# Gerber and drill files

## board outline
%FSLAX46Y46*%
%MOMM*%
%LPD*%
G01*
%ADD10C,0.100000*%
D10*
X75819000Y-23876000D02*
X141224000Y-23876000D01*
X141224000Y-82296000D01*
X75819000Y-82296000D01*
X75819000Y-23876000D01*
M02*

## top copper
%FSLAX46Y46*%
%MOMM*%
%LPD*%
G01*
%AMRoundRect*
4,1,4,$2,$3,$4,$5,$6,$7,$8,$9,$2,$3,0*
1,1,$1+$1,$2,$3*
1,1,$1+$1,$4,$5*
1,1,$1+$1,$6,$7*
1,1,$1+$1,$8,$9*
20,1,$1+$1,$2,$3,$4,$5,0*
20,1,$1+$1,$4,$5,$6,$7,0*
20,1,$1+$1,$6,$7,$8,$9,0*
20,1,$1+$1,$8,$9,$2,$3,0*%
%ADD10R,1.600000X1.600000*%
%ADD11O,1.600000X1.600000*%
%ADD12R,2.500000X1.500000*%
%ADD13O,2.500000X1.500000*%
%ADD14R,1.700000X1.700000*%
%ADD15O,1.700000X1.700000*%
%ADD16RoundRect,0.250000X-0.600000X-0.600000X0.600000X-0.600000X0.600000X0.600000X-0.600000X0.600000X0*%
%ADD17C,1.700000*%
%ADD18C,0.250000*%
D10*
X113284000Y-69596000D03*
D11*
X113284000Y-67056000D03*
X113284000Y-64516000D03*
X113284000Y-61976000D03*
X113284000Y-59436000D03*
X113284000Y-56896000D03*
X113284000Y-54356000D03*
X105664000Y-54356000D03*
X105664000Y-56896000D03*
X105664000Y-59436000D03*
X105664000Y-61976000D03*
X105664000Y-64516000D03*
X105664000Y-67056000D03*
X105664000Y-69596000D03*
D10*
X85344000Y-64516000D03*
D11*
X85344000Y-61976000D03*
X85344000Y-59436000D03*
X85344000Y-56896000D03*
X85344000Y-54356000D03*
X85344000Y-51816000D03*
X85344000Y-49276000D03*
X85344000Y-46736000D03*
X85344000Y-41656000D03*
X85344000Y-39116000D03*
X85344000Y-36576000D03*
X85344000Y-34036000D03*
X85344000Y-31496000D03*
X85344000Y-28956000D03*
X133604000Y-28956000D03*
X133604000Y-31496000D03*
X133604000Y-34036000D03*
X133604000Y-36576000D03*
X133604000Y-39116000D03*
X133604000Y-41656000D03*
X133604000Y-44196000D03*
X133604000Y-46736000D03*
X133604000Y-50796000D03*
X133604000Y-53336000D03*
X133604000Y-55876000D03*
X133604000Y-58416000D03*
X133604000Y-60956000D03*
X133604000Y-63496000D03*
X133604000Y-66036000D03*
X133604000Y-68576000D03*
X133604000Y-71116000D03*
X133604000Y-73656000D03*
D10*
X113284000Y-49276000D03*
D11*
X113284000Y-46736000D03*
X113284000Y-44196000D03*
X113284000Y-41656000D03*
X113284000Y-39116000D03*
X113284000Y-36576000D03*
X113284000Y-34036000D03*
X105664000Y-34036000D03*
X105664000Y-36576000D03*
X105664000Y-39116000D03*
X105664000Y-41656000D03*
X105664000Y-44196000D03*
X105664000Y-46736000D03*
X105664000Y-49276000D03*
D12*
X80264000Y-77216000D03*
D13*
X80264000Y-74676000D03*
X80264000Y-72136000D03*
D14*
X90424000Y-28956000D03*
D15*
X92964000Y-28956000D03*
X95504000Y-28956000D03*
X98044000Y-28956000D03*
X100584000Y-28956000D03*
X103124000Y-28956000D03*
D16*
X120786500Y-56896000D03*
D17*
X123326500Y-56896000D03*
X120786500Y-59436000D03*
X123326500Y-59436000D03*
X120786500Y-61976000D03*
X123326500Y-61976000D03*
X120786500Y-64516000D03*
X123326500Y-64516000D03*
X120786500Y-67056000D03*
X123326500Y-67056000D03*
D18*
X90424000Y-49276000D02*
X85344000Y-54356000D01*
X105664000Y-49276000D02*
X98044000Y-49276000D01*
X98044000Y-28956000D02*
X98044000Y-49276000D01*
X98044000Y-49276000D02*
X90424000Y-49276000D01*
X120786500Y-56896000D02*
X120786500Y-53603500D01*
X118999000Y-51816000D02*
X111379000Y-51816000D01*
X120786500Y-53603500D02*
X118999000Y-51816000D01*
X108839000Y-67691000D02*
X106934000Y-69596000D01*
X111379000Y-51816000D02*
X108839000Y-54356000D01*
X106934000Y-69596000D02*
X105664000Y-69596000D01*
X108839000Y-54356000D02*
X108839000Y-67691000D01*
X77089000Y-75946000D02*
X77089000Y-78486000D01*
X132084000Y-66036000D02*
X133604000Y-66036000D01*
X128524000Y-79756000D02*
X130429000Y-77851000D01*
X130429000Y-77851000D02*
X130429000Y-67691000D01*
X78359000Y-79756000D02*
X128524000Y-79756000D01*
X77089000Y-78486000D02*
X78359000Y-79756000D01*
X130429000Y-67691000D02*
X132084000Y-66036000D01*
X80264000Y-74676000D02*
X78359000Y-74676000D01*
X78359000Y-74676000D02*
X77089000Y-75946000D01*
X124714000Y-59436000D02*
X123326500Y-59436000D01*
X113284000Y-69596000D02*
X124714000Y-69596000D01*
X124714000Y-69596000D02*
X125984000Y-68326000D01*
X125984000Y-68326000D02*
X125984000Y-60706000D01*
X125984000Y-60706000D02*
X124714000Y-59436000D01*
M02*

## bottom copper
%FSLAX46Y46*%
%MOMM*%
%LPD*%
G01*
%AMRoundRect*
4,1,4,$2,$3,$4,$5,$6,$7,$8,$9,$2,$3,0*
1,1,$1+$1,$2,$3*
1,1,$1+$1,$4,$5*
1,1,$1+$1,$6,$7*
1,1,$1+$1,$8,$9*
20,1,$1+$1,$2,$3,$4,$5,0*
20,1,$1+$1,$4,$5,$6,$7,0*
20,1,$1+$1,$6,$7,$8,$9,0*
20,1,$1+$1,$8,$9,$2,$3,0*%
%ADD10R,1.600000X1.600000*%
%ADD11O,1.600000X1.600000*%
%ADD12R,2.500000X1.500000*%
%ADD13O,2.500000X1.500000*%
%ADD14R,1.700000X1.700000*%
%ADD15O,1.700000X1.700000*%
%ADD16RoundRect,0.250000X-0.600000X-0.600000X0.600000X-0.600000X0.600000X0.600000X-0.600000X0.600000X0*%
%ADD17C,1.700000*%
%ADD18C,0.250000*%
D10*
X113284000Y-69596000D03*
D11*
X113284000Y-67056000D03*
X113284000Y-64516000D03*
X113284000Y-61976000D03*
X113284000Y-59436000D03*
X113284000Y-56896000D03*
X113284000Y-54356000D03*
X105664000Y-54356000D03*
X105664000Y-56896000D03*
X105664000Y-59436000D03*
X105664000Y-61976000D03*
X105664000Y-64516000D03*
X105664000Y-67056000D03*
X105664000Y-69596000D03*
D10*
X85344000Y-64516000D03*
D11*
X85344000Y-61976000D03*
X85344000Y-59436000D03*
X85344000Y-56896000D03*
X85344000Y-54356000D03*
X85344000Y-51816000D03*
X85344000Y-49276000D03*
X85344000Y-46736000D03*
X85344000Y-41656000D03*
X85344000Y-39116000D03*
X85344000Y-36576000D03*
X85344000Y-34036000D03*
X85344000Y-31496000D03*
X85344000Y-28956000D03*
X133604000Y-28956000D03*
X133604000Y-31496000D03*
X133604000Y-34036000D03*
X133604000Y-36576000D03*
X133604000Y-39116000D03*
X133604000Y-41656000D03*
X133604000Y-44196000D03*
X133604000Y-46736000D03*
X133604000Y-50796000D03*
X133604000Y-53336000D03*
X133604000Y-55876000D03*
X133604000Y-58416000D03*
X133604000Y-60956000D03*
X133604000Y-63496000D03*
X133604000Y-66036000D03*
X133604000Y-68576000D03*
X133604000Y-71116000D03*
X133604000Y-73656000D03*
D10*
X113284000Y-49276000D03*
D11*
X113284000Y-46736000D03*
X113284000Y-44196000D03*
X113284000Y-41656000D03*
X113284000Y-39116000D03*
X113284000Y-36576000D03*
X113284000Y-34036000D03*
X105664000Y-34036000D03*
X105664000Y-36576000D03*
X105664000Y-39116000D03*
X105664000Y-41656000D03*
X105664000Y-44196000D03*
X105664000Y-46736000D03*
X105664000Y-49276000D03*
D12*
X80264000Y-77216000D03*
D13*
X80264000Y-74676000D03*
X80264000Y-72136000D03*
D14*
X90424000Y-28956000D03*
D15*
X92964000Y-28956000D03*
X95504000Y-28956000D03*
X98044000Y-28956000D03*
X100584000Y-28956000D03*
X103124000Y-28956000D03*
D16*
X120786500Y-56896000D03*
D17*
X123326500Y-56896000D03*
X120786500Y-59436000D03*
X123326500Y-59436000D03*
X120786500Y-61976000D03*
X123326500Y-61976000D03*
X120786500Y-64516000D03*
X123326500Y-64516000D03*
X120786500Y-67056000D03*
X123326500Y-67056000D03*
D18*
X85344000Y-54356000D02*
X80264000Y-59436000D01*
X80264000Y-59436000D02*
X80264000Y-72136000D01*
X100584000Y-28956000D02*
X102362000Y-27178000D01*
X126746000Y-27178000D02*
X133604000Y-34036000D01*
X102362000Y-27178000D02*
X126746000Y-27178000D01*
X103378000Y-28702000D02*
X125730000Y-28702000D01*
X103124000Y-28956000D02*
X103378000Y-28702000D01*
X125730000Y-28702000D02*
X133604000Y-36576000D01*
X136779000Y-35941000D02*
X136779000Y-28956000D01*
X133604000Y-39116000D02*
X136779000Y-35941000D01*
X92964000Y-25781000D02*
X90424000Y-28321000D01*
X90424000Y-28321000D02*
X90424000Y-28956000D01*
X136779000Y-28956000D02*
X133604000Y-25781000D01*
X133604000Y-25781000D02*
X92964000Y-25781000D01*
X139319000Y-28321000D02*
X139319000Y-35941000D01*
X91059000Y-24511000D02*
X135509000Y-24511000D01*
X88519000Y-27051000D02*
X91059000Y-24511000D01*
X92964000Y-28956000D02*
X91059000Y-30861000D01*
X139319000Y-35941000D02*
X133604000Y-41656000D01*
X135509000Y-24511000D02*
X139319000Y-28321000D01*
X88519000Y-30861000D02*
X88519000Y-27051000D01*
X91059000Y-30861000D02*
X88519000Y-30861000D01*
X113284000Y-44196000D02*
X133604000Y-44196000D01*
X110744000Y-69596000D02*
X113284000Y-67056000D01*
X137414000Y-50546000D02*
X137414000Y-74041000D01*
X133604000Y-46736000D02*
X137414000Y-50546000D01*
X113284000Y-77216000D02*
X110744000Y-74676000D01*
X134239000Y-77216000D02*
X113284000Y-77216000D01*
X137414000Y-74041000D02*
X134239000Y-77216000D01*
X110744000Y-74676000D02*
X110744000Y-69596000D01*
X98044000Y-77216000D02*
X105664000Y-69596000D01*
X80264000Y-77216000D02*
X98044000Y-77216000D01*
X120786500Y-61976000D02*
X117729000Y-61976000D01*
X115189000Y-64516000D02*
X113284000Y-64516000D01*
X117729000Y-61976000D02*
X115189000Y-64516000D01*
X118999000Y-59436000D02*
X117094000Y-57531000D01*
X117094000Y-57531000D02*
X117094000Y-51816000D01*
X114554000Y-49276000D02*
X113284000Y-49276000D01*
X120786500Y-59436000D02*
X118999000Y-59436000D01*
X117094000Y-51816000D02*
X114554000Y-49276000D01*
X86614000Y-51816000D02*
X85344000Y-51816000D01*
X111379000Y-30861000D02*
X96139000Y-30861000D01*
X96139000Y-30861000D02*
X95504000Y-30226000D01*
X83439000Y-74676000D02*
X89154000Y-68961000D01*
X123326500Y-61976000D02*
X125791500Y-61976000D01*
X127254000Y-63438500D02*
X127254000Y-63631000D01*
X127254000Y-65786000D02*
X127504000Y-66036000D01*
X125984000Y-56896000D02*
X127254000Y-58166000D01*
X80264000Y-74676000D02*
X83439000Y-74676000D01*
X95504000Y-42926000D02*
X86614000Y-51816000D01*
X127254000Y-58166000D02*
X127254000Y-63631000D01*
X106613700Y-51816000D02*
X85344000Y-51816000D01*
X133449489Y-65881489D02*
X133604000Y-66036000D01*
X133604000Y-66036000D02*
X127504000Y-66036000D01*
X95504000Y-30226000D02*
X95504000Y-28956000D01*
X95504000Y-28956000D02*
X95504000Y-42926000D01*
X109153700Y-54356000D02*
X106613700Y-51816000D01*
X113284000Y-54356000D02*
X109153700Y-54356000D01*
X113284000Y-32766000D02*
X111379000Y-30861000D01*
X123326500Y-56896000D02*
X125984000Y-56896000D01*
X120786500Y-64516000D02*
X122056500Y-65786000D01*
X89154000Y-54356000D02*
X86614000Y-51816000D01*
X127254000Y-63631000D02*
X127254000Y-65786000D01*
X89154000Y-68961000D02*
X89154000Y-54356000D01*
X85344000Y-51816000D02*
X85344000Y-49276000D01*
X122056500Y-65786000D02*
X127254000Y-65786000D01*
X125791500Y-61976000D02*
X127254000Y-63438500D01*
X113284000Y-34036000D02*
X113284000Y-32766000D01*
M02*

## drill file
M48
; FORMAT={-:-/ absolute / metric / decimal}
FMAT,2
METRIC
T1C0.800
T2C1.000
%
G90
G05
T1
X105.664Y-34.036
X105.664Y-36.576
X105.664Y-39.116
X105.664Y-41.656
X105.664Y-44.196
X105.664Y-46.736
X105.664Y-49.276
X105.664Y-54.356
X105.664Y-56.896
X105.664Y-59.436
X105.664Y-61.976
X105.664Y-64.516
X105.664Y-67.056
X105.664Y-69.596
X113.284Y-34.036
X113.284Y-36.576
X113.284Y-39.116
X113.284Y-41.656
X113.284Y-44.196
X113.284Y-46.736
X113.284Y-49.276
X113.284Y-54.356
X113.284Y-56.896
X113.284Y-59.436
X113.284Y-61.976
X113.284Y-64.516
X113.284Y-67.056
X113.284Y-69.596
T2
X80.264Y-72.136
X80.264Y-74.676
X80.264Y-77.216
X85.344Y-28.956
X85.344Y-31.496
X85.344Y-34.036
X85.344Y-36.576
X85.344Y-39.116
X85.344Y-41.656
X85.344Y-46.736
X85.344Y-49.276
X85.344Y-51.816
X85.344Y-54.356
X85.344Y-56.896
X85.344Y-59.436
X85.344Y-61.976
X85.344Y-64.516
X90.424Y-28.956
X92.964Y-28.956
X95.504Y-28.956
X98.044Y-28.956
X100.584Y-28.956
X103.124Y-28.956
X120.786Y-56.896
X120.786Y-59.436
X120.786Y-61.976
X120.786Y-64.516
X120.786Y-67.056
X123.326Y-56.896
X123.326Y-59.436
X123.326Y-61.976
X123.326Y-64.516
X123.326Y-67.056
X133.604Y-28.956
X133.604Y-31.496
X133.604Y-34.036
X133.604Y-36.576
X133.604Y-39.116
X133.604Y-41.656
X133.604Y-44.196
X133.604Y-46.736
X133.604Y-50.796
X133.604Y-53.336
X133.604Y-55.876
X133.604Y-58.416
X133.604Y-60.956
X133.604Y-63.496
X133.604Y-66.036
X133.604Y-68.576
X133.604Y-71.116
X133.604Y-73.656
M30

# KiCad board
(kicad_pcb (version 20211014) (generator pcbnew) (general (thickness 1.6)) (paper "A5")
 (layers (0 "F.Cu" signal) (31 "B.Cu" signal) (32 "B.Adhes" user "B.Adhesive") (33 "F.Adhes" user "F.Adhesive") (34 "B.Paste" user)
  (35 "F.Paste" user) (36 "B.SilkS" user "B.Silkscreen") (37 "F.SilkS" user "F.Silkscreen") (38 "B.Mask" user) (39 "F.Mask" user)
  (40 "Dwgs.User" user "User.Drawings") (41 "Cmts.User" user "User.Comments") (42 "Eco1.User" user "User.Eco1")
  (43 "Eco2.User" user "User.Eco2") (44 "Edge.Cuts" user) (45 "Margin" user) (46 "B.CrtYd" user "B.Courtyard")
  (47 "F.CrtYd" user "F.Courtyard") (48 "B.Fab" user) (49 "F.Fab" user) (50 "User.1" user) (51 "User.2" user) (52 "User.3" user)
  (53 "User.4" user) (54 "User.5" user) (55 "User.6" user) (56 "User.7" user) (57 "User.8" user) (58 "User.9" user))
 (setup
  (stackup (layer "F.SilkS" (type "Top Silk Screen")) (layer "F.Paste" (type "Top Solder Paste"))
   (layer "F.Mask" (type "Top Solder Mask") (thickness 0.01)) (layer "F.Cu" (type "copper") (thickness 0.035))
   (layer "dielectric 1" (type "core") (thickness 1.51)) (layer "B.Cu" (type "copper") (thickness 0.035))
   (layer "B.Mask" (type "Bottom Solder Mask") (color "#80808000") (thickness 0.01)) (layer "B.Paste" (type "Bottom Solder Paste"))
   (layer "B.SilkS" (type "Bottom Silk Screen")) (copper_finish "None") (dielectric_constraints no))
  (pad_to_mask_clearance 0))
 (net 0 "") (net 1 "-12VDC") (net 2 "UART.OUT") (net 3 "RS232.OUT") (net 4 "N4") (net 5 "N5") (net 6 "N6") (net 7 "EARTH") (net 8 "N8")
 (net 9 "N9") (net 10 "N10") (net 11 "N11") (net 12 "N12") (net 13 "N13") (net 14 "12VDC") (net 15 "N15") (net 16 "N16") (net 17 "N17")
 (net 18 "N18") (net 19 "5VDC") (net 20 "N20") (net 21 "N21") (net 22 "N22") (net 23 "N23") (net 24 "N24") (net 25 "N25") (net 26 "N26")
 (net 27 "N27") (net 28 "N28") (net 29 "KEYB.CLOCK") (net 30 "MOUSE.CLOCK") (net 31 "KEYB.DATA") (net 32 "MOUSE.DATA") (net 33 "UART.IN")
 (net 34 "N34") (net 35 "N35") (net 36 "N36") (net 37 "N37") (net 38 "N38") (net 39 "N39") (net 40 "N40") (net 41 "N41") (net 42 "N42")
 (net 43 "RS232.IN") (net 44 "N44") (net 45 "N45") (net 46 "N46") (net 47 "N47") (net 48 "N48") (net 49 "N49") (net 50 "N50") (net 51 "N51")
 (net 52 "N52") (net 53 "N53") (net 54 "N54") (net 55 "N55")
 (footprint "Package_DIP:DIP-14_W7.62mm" (layer "F.Cu") (at 113.284 69.596 180)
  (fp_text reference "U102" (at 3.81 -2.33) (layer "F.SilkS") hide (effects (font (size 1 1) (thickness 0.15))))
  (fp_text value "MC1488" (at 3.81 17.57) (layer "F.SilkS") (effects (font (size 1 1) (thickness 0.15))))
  (pad "1" thru_hole rect (at 0 0 180) (size 1.6 1.6) (drill 0.8) (layers *.Cu *.Mask) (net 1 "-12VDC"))
  (pad "2" thru_hole oval (at 0 2.54 180) (size 1.6 1.6) (drill 0.8) (layers *.Cu *.Mask) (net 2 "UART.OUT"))
  (pad "3" thru_hole oval (at 0 5.08 180) (size 1.6 1.6) (drill 0.8) (layers *.Cu *.Mask) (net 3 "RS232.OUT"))
  (pad "4" thru_hole oval (at 0 7.62 180) (size 1.6 1.6) (drill 0.8) (layers *.Cu *.Mask) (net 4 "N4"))
  (pad "5" thru_hole oval (at 0 10.16 180) (size 1.6 1.6) (drill 0.8) (layers *.Cu *.Mask) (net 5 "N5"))
  (pad "6" thru_hole oval (at 0 12.7 180) (size 1.6 1.6) (drill 0.8) (layers *.Cu *.Mask) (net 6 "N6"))
  (pad "7" thru_hole oval (at 0 15.24 180) (size 1.6 1.6) (drill 0.8) (layers *.Cu *.Mask) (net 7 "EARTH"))
  (pad "8" thru_hole oval (at 7.62 15.24 180) (size 1.6 1.6) (drill 0.8) (layers *.Cu *.Mask) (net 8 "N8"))
  (pad "9" thru_hole oval (at 7.62 12.7 180) (size 1.6 1.6) (drill 0.8) (layers *.Cu *.Mask) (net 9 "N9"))
  (pad "10" thru_hole oval (at 7.62 10.16 180) (size 1.6 1.6) (drill 0.8) (layers *.Cu *.Mask) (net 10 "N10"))
  (pad "11" thru_hole oval (at 7.62 7.62 180) (size 1.6 1.6) (drill 0.8) (layers *.Cu *.Mask) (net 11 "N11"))
  (pad "12" thru_hole oval (at 7.62 5.08 180) (size 1.6 1.6) (drill 0.8) (layers *.Cu *.Mask) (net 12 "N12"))
  (pad "13" thru_hole oval (at 7.62 2.54 180) (size 1.6 1.6) (drill 0.8) (layers *.Cu *.Mask) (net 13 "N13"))
  (pad "14" thru_hole oval (at 7.62 0 180) (size 1.6 1.6) (drill 0.8) (layers *.Cu *.Mask) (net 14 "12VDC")))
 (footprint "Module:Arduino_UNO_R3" (layer "F.Cu") (at 85.344 64.516 90)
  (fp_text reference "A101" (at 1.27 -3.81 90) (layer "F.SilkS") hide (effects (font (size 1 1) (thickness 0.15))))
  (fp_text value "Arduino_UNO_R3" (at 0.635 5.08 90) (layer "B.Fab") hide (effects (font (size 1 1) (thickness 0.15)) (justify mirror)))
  (pad "1" thru_hole rect (at 0 0 180) (size 1.6 1.6) (drill 1) (layers *.Cu *.Mask) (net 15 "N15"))
  (pad "2" thru_hole oval (at 2.54 0 180) (size 1.6 1.6) (drill 1) (layers *.Cu *.Mask) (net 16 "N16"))
  (pad "3" thru_hole oval (at 5.08 0 180) (size 1.6 1.6) (drill 1) (layers *.Cu *.Mask) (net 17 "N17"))
  (pad "4" thru_hole oval (at 7.62 0 180) (size 1.6 1.6) (drill 1) (layers *.Cu *.Mask) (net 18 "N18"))
  (pad "5" thru_hole oval (at 10.16 0 180) (size 1.6 1.6) (drill 1) (layers *.Cu *.Mask) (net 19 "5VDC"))
  (pad "6" thru_hole oval (at 12.7 0 180) (size 1.6 1.6) (drill 1) (layers *.Cu *.Mask) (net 7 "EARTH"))
  (pad "7" thru_hole oval (at 15.24 0 180) (size 1.6 1.6) (drill 1) (layers *.Cu *.Mask) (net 7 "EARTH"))
  (pad "8" thru_hole oval (at 17.78 0 180) (size 1.6 1.6) (drill 1) (layers *.Cu *.Mask) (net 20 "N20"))
  (pad "9" thru_hole oval (at 22.86 0 180) (size 1.6 1.6) (drill 1) (layers *.Cu *.Mask) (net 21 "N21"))
  (pad "10" thru_hole oval (at 25.4 0 180) (size 1.6 1.6) (drill 1) (layers *.Cu *.Mask) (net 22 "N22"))
  (pad "11" thru_hole oval (at 27.94 0 180) (size 1.6 1.6) (drill 1) (layers *.Cu *.Mask) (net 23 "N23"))
  (pad "12" thru_hole oval (at 30.48 0 180) (size 1.6 1.6) (drill 1) (layers *.Cu *.Mask) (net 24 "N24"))
  (pad "13" thru_hole oval (at 33.02 0 180) (size 1.6 1.6) (drill 1) (layers *.Cu *.Mask) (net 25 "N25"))
  (pad "14" thru_hole oval (at 35.56 0 180) (size 1.6 1.6) (drill 1) (layers *.Cu *.Mask) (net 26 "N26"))
  (pad "15" thru_hole oval (at 35.56 48.26 180) (size 1.6 1.6) (drill 1) (layers *.Cu *.Mask) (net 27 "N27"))
  (pad "16" thru_hole oval (at 33.02 48.26 180) (size 1.6 1.6) (drill 1) (layers *.Cu *.Mask) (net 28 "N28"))
  (pad "17" thru_hole oval (at 30.48 48.26 180) (size 1.6 1.6) (drill 1) (layers *.Cu *.Mask) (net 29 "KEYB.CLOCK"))
  (pad "18" thru_hole oval (at 27.94 48.26 180) (size 1.6 1.6) (drill 1) (layers *.Cu *.Mask) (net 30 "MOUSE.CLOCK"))
  (pad "19" thru_hole oval (at 25.4 48.26 180) (size 1.6 1.6) (drill 1) (layers *.Cu *.Mask) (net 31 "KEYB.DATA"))
  (pad "20" thru_hole oval (at 22.86 48.26 180) (size 1.6 1.6) (drill 1) (layers *.Cu *.Mask) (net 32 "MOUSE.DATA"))
  (pad "21" thru_hole oval (at 20.32 48.26 180) (size 1.6 1.6) (drill 1) (layers *.Cu *.Mask) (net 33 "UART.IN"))
  (pad "22" thru_hole oval (at 17.78 48.26 180) (size 1.6 1.6) (drill 1) (layers *.Cu *.Mask) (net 2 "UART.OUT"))
  (pad "23" thru_hole oval (at 13.72 48.26 180) (size 1.6 1.6) (drill 1) (layers *.Cu *.Mask) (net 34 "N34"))
  (pad "24" thru_hole oval (at 11.18 48.26 180) (size 1.6 1.6) (drill 1) (layers *.Cu *.Mask) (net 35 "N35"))
  (pad "25" thru_hole oval (at 8.64 48.26 180) (size 1.6 1.6) (drill 1) (layers *.Cu *.Mask) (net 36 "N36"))
  (pad "26" thru_hole oval (at 6.1 48.26 180) (size 1.6 1.6) (drill 1) (layers *.Cu *.Mask) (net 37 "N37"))
  (pad "27" thru_hole oval (at 3.56 48.26 180) (size 1.6 1.6) (drill 1) (layers *.Cu *.Mask) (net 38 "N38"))
  (pad "28" thru_hole oval (at 1.02 48.26 180) (size 1.6 1.6) (drill 1) (layers *.Cu *.Mask) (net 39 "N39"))
  (pad "29" thru_hole oval (at -1.52 48.26 180) (size 1.6 1.6) (drill 1) (layers *.Cu *.Mask) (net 7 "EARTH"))
  (pad "30" thru_hole oval (at -4.06 48.26 180) (size 1.6 1.6) (drill 1) (layers *.Cu *.Mask) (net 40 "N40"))
  (pad "31" thru_hole oval (at -6.6 48.26 180) (size 1.6 1.6) (drill 1) (layers *.Cu *.Mask) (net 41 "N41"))
  (pad "32" thru_hole oval (at -9.14 48.26 180) (size 1.6 1.6) (drill 1) (layers *.Cu *.Mask) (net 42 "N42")))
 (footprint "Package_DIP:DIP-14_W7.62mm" (layer "F.Cu") (at 113.284 49.276 180)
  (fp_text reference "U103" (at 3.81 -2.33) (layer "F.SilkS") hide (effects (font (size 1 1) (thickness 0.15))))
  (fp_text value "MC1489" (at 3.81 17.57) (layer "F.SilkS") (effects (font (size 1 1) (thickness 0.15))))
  (pad "1" thru_hole rect (at 0 0 180) (size 1.6 1.6) (drill 0.8) (layers *.Cu *.Mask) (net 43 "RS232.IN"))
  (pad "2" thru_hole oval (at 0 2.54 180) (size 1.6 1.6) (drill 0.8) (layers *.Cu *.Mask) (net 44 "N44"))
  (pad "3" thru_hole oval (at 0 5.08 180) (size 1.6 1.6) (drill 0.8) (layers *.Cu *.Mask) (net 33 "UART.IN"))
  (pad "4" thru_hole oval (at 0 7.62 180) (size 1.6 1.6) (drill 0.8) (layers *.Cu *.Mask) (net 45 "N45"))
  (pad "5" thru_hole oval (at 0 10.16 180) (size 1.6 1.6) (drill 0.8) (layers *.Cu *.Mask) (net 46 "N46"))
  (pad "6" thru_hole oval (at 0 12.7 180) (size 1.6 1.6) (drill 0.8) (layers *.Cu *.Mask) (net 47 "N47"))
  (pad "7" thru_hole oval (at 0 15.24 180) (size 1.6 1.6) (drill 0.8) (layers *.Cu *.Mask) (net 7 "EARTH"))
  (pad "8" thru_hole oval (at 7.62 15.24 180) (size 1.6 1.6) (drill 0.8) (layers *.Cu *.Mask) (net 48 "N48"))
  (pad "9" thru_hole oval (at 7.62 12.7 180) (size 1.6 1.6) (drill 0.8) (layers *.Cu *.Mask) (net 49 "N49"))
  (pad "10" thru_hole oval (at 7.62 10.16 180) (size 1.6 1.6) (drill 0.8) (layers *.Cu *.Mask) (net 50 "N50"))
  (pad "11" thru_hole oval (at 7.62 7.62 180) (size 1.6 1.6) (drill 0.8) (layers *.Cu *.Mask) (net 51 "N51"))
  (pad "12" thru_hole oval (at 7.62 5.08 180) (size 1.6 1.6) (drill 0.8) (layers *.Cu *.Mask) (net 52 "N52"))
  (pad "13" thru_hole oval (at 7.62 2.54 180) (size 1.6 1.6) (drill 0.8) (layers *.Cu *.Mask) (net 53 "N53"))
  (pad "14" thru_hole oval (at 7.62 0 180) (size 1.6 1.6) (drill 0.8) (layers *.Cu *.Mask) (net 19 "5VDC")))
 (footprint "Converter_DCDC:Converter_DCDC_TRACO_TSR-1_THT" (layer "F.Cu") (at 80.264 77.216 90)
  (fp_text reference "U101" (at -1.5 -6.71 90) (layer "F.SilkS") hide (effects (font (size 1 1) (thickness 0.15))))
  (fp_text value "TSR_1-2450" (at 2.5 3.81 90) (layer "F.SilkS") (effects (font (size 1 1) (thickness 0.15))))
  (pad "1" thru_hole rect (at 0 0 90) (size 1.5 2.5) (drill 1) (layers *.Cu *.Mask) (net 14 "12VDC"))
  (pad "2" thru_hole oval (at 2.54 0 90) (size 1.5 2.5) (drill 1) (layers *.Cu *.Mask) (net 7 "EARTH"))
  (pad "3" thru_hole oval (at 5.08 0 90) (size 1.5 2.5) (drill 1) (layers *.Cu *.Mask) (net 19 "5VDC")))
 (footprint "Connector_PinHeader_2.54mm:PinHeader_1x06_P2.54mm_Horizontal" (layer "F.Cu") (at 90.424 28.956 90)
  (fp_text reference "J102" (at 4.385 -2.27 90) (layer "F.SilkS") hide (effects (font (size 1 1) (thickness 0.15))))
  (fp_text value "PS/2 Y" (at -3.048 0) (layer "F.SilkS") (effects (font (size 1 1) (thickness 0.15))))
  (pad "1" thru_hole rect (at 0 0 90) (size 1.7 1.7) (drill 1) (layers *.Cu *.Mask) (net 31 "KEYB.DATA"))
  (pad "2" thru_hole oval (at 0 2.54 90) (size 1.7 1.7) (drill 1) (layers *.Cu *.Mask) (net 32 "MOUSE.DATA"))
  (pad "3" thru_hole oval (at 0 5.08 90) (size 1.7 1.7) (drill 1) (layers *.Cu *.Mask) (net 7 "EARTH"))
  (pad "4" thru_hole oval (at 0 7.62 90) (size 1.7 1.7) (drill 1) (layers *.Cu *.Mask) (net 19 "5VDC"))
  (pad "5" thru_hole oval (at 0 10.16 90) (size 1.7 1.7) (drill 1) (layers *.Cu *.Mask) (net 29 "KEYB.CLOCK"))
  (pad "6" thru_hole oval (at 0 12.7 90) (size 1.7 1.7) (drill 1) (layers *.Cu *.Mask) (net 30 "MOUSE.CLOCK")))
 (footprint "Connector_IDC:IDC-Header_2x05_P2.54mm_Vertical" (layer "F.Cu") (at 120.7865 56.896)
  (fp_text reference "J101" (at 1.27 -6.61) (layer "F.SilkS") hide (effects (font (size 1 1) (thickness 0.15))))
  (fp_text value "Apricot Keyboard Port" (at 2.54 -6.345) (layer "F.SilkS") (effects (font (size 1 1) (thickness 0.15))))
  (pad "1" thru_hole roundrect (at 0 0) (size 1.7 1.7) (drill 1) (layers *.Cu *.Mask) (roundrect_rratio 0.147059) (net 14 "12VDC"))
  (pad "2" thru_hole circle (at 2.54 0) (size 1.7 1.7) (drill 1) (layers *.Cu *.Mask) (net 7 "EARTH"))
  (pad "3" thru_hole circle (at 0 2.54) (size 1.7 1.7) (drill 1) (layers *.Cu *.Mask) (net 43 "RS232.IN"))
  (pad "4" thru_hole circle (at 2.54 2.54) (size 1.7 1.7) (drill 1) (layers *.Cu *.Mask) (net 1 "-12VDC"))
  (pad "5" thru_hole circle (at 0 5.08) (size 1.7 1.7) (drill 1) (layers *.Cu *.Mask) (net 3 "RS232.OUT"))
  (pad "6" thru_hole circle (at 2.54 5.08) (size 1.7 1.7) (drill 1) (layers *.Cu *.Mask) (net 7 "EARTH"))
  (pad "7" thru_hole circle (at 0 7.62) (size 1.7 1.7) (drill 1) (layers *.Cu *.Mask) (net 7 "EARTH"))
  (pad "8" thru_hole circle (at 2.54 7.62) (size 1.7 1.7) (drill 1) (layers *.Cu *.Mask) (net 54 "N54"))
  (pad "9" thru_hole circle (at 0 10.16) (size 1.7 1.7) (drill 1) (layers *.Cu *.Mask) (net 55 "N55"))
  (pad "10" thru_hole circle (at 2.54 10.16) (size 1.7 1.7) (drill 1) (layers *.Cu *.Mask)))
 (gr_rect (start 141.224 82.296) (end 75.819 23.876) (layer "Edge.Cuts") (width 0.1) (fill none))
 (segment (start 90.424 49.276) (end 85.344 54.356) (width 0.25) (layer "F.Cu") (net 19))
 (segment (start 105.664 49.276) (end 98.044 49.276) (width 0.25) (layer "F.Cu") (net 19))
 (segment (start 98.044 28.956) (end 98.044 49.276) (width 0.25) (layer "F.Cu") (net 19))
 (segment (start 98.044 49.276) (end 90.424 49.276) (width 0.25) (layer "F.Cu") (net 19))
 (segment (start 85.344 54.356) (end 80.264 59.436) (width 0.25) (layer "B.Cu") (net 19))
 (segment (start 80.264 59.436) (end 80.264 72.136) (width 0.25) (layer "B.Cu") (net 19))
 (segment (start 100.584 28.956) (end 102.362 27.178) (width 0.25) (layer "B.Cu") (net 29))
 (segment (start 126.746 27.178) (end 133.604 34.036) (width 0.25) (layer "B.Cu") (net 29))
 (segment (start 102.362 27.178) (end 126.746 27.178) (width 0.25) (layer "B.Cu") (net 29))
 (segment (start 103.378 28.702) (end 125.73 28.702) (width 0.25) (layer "B.Cu") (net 30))
 (segment (start 103.124 28.956) (end 103.378 28.702) (width 0.25) (layer "B.Cu") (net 30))
 (segment (start 125.73 28.702) (end 133.604 36.576) (width 0.25) (layer "B.Cu") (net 30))
 (segment (start 136.779 35.941) (end 136.779 28.956) (width 0.25) (layer "B.Cu") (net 31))
 (segment (start 133.604 39.116) (end 136.779 35.941) (width 0.25) (layer "B.Cu") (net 31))
 (segment (start 92.964 25.781) (end 90.424 28.321) (width 0.25) (layer "B.Cu") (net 31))
 (segment (start 90.424 28.321) (end 90.424 28.956) (width 0.25) (layer "B.Cu") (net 31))
 (segment (start 136.779 28.956) (end 133.604 25.781) (width 0.25) (layer "B.Cu") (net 31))
 (segment (start 133.604 25.781) (end 92.964 25.781) (width 0.25) (layer "B.Cu") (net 31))
 (segment (start 139.319 28.321) (end 139.319 35.941) (width 0.25) (layer "B.Cu") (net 32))
 (segment (start 91.059 24.511) (end 135.509 24.511) (width 0.25) (layer "B.Cu") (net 32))
 (segment (start 88.519 27.051) (end 91.059 24.511) (width 0.25) (layer "B.Cu") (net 32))
 (segment (start 92.964 28.956) (end 91.059 30.861) (width 0.25) (layer "B.Cu") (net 32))
 (segment (start 139.319 35.941) (end 133.604 41.656) (width 0.25) (layer "B.Cu") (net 32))
 (segment (start 135.509 24.511) (end 139.319 28.321) (width 0.25) (layer "B.Cu") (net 32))
 (segment (start 88.519 30.861) (end 88.519 27.051) (width 0.25) (layer "B.Cu") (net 32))
 (segment (start 91.059 30.861) (end 88.519 30.861) (width 0.25) (layer "B.Cu") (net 32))
 (segment (start 113.284 44.196) (end 133.604 44.196) (width 0.25) (layer "B.Cu") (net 33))
 (segment (start 110.744 69.596) (end 113.284 67.056) (width 0.25) (layer "B.Cu") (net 2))
 (segment (start 137.414 50.546) (end 137.414 74.041) (width 0.25) (layer "B.Cu") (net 2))
 (segment (start 133.604 46.736) (end 137.414 50.546) (width 0.25) (layer "B.Cu") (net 2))
 (segment (start 113.284 77.216) (end 110.744 74.676) (width 0.25) (layer "B.Cu") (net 2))
 (segment (start 134.239 77.216) (end 113.284 77.216) (width 0.25) (layer "B.Cu") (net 2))
 (segment (start 137.414 74.041) (end 134.239 77.216) (width 0.25) (layer "B.Cu") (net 2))
 (segment (start 110.744 74.676) (end 110.744 69.596) (width 0.25) (layer "B.Cu") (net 2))
 (segment (start 120.7865 56.896) (end 120.7865 53.6035) (width 0.25) (layer "F.Cu") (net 14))
 (segment (start 118.999 51.816) (end 111.379 51.816) (width 0.25) (layer "F.Cu") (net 14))
 (segment (start 120.7865 53.6035) (end 118.999 51.816) (width 0.25) (layer "F.Cu") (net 14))
 (segment (start 108.839 67.691) (end 106.934 69.596) (width 0.25) (layer "F.Cu") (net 14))
 (segment (start 111.379 51.816) (end 108.839 54.356) (width 0.25) (layer "F.Cu") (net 14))
 (segment (start 106.934 69.596) (end 105.664 69.596) (width 0.25) (layer "F.Cu") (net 14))
 (segment (start 108.839 54.356) (end 108.839 67.691) (width 0.25) (layer "F.Cu") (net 14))
 (segment (start 98.044 77.216) (end 105.664 69.596) (width 0.25) (layer "B.Cu") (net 14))
 (segment (start 80.264 77.216) (end 98.044 77.216) (width 0.25) (layer "B.Cu") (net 14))
 (segment (start 120.7865 61.976) (end 117.729 61.976) (width 0.25) (layer "B.Cu") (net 3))
 (segment (start 115.189 64.516) (end 113.284 64.516) (width 0.25) (layer "B.Cu") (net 3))
 (segment (start 117.729 61.976) (end 115.189 64.516) (width 0.25) (layer "B.Cu") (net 3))
 (segment (start 118.999 59.436) (end 117.094 57.531) (width 0.25) (layer "B.Cu") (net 43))
 (segment (start 117.094 57.531) (end 117.094 51.816) (width 0.25) (layer "B.Cu") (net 43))
 (segment (start 114.554 49.276) (end 113.284 49.276) (width 0.25) (layer "B.Cu") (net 43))
 (segment (start 120.7865 59.436) (end 118.999 59.436) (width 0.25) (layer "B.Cu") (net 43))
 (segment (start 117.094 51.816) (end 114.554 49.276) (width 0.25) (layer "B.Cu") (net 43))
 (segment (start 77.089 75.946) (end 77.089 78.486) (width 0.25) (layer "F.Cu") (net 7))
 (segment (start 132.084 66.036) (end 133.604 66.036) (width 0.25) (layer "F.Cu") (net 7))
 (segment (start 128.524 79.756) (end 130.429 77.851) (width 0.25) (layer "F.Cu") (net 7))
 (segment (start 130.429 77.851) (end 130.429 67.691) (width 0.25) (layer "F.Cu") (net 7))
 (segment (start 78.359 79.756) (end 128.524 79.756) (width 0.25) (layer "F.Cu") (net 7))
 (segment (start 77.089 78.486) (end 78.359 79.756) (width 0.25) (layer "F.Cu") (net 7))
 (segment (start 130.429 67.691) (end 132.084 66.036) (width 0.25) (layer "F.Cu") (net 7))
 (segment (start 80.264 74.676) (end 78.359 74.676) (width 0.25) (layer "F.Cu") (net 7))
 (segment (start 78.359 74.676) (end 77.089 75.946) (width 0.25) (layer "F.Cu") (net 7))
 (segment (start 86.614 51.816) (end 85.344 51.816) (width 0.25) (layer "B.Cu") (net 7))
 (segment (start 111.379 30.861) (end 96.139 30.861) (width 0.25) (layer "B.Cu") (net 7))
 (segment (start 96.139 30.861) (end 95.504 30.226) (width 0.25) (layer "B.Cu") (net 7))
 (segment (start 83.439 74.676) (end 89.154 68.961) (width 0.25) (layer "B.Cu") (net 7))
 (segment (start 123.3265 61.976) (end 125.7915 61.976) (width 0.25) (layer "B.Cu") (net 7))
 (segment (start 127.254 63.4385) (end 127.254 63.631) (width 0.25) (layer "B.Cu") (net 7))
 (segment (start 127.254 65.786) (end 127.504 66.036) (width 0.25) (layer "B.Cu") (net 7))
 (segment (start 125.984 56.896) (end 127.254 58.166) (width 0.25) (layer "B.Cu") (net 7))
 (segment (start 80.264 74.676) (end 83.439 74.676) (width 0.25) (layer "B.Cu") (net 7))
 (segment (start 95.504 42.926) (end 86.614 51.816) (width 0.25) (layer "B.Cu") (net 7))
 (segment (start 127.254 58.166) (end 127.254 63.631) (width 0.25) (layer "B.Cu") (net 7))
 (segment (start 106.6137 51.816) (end 85.344 51.816) (width 0.25) (layer "B.Cu") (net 7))
 (segment (start 133.449489 65.881489) (end 133.604 66.036) (width 0.25) (layer "B.Cu") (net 7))
 (segment (start 133.604 66.036) (end 127.504 66.036) (width 0.25) (layer "B.Cu") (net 7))
 (segment (start 95.504 30.226) (end 95.504 28.956) (width 0.25) (layer "B.Cu") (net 7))
 (segment (start 95.504 28.956) (end 95.504 42.926) (width 0.25) (layer "B.Cu") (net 7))
 (segment (start 109.1537 54.356) (end 106.6137 51.816) (width 0.25) (layer "B.Cu") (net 7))
 (segment (start 113.284 54.356) (end 109.1537 54.356) (width 0.25) (layer "B.Cu") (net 7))
 (segment (start 113.284 32.766) (end 111.379 30.861) (width 0.25) (layer "B.Cu") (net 7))
 (segment (start 123.3265 56.896) (end 125.984 56.896) (width 0.25) (layer "B.Cu") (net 7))
 (segment (start 120.7865 64.516) (end 122.0565 65.786) (width 0.25) (layer "B.Cu") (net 7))
 (segment (start 89.154 54.356) (end 86.614 51.816) (width 0.25) (layer "B.Cu") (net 7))
 (segment (start 127.254 63.631) (end 127.254 65.786) (width 0.25) (layer "B.Cu") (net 7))
 (segment (start 89.154 68.961) (end 89.154 54.356) (width 0.25) (layer "B.Cu") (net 7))
 (segment (start 85.344 51.816) (end 85.344 49.276) (width 0.25) (layer "B.Cu") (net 7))
 (segment (start 122.0565 65.786) (end 127.254 65.786) (width 0.25) (layer "B.Cu") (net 7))
 (segment (start 125.7915 61.976) (end 127.254 63.4385) (width 0.25) (layer "B.Cu") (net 7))
 (segment (start 113.284 34.036) (end 113.284 32.766) (width 0.25) (layer "B.Cu") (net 7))
 (segment (start 124.714 59.436) (end 123.3265 59.436) (width 0.25) (layer "F.Cu") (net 1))
 (segment (start 113.284 69.596) (end 124.714 69.596) (width 0.25) (layer "F.Cu") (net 1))
 (segment (start 124.714 69.596) (end 125.984 68.326) (width 0.25) (layer "F.Cu") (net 1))
 (segment (start 125.984 68.326) (end 125.984 60.706) (width 0.25) (layer "F.Cu") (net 1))
 (segment (start 125.984 60.706) (end 124.714 59.436) (width 0.25) (layer "F.Cu") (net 1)))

